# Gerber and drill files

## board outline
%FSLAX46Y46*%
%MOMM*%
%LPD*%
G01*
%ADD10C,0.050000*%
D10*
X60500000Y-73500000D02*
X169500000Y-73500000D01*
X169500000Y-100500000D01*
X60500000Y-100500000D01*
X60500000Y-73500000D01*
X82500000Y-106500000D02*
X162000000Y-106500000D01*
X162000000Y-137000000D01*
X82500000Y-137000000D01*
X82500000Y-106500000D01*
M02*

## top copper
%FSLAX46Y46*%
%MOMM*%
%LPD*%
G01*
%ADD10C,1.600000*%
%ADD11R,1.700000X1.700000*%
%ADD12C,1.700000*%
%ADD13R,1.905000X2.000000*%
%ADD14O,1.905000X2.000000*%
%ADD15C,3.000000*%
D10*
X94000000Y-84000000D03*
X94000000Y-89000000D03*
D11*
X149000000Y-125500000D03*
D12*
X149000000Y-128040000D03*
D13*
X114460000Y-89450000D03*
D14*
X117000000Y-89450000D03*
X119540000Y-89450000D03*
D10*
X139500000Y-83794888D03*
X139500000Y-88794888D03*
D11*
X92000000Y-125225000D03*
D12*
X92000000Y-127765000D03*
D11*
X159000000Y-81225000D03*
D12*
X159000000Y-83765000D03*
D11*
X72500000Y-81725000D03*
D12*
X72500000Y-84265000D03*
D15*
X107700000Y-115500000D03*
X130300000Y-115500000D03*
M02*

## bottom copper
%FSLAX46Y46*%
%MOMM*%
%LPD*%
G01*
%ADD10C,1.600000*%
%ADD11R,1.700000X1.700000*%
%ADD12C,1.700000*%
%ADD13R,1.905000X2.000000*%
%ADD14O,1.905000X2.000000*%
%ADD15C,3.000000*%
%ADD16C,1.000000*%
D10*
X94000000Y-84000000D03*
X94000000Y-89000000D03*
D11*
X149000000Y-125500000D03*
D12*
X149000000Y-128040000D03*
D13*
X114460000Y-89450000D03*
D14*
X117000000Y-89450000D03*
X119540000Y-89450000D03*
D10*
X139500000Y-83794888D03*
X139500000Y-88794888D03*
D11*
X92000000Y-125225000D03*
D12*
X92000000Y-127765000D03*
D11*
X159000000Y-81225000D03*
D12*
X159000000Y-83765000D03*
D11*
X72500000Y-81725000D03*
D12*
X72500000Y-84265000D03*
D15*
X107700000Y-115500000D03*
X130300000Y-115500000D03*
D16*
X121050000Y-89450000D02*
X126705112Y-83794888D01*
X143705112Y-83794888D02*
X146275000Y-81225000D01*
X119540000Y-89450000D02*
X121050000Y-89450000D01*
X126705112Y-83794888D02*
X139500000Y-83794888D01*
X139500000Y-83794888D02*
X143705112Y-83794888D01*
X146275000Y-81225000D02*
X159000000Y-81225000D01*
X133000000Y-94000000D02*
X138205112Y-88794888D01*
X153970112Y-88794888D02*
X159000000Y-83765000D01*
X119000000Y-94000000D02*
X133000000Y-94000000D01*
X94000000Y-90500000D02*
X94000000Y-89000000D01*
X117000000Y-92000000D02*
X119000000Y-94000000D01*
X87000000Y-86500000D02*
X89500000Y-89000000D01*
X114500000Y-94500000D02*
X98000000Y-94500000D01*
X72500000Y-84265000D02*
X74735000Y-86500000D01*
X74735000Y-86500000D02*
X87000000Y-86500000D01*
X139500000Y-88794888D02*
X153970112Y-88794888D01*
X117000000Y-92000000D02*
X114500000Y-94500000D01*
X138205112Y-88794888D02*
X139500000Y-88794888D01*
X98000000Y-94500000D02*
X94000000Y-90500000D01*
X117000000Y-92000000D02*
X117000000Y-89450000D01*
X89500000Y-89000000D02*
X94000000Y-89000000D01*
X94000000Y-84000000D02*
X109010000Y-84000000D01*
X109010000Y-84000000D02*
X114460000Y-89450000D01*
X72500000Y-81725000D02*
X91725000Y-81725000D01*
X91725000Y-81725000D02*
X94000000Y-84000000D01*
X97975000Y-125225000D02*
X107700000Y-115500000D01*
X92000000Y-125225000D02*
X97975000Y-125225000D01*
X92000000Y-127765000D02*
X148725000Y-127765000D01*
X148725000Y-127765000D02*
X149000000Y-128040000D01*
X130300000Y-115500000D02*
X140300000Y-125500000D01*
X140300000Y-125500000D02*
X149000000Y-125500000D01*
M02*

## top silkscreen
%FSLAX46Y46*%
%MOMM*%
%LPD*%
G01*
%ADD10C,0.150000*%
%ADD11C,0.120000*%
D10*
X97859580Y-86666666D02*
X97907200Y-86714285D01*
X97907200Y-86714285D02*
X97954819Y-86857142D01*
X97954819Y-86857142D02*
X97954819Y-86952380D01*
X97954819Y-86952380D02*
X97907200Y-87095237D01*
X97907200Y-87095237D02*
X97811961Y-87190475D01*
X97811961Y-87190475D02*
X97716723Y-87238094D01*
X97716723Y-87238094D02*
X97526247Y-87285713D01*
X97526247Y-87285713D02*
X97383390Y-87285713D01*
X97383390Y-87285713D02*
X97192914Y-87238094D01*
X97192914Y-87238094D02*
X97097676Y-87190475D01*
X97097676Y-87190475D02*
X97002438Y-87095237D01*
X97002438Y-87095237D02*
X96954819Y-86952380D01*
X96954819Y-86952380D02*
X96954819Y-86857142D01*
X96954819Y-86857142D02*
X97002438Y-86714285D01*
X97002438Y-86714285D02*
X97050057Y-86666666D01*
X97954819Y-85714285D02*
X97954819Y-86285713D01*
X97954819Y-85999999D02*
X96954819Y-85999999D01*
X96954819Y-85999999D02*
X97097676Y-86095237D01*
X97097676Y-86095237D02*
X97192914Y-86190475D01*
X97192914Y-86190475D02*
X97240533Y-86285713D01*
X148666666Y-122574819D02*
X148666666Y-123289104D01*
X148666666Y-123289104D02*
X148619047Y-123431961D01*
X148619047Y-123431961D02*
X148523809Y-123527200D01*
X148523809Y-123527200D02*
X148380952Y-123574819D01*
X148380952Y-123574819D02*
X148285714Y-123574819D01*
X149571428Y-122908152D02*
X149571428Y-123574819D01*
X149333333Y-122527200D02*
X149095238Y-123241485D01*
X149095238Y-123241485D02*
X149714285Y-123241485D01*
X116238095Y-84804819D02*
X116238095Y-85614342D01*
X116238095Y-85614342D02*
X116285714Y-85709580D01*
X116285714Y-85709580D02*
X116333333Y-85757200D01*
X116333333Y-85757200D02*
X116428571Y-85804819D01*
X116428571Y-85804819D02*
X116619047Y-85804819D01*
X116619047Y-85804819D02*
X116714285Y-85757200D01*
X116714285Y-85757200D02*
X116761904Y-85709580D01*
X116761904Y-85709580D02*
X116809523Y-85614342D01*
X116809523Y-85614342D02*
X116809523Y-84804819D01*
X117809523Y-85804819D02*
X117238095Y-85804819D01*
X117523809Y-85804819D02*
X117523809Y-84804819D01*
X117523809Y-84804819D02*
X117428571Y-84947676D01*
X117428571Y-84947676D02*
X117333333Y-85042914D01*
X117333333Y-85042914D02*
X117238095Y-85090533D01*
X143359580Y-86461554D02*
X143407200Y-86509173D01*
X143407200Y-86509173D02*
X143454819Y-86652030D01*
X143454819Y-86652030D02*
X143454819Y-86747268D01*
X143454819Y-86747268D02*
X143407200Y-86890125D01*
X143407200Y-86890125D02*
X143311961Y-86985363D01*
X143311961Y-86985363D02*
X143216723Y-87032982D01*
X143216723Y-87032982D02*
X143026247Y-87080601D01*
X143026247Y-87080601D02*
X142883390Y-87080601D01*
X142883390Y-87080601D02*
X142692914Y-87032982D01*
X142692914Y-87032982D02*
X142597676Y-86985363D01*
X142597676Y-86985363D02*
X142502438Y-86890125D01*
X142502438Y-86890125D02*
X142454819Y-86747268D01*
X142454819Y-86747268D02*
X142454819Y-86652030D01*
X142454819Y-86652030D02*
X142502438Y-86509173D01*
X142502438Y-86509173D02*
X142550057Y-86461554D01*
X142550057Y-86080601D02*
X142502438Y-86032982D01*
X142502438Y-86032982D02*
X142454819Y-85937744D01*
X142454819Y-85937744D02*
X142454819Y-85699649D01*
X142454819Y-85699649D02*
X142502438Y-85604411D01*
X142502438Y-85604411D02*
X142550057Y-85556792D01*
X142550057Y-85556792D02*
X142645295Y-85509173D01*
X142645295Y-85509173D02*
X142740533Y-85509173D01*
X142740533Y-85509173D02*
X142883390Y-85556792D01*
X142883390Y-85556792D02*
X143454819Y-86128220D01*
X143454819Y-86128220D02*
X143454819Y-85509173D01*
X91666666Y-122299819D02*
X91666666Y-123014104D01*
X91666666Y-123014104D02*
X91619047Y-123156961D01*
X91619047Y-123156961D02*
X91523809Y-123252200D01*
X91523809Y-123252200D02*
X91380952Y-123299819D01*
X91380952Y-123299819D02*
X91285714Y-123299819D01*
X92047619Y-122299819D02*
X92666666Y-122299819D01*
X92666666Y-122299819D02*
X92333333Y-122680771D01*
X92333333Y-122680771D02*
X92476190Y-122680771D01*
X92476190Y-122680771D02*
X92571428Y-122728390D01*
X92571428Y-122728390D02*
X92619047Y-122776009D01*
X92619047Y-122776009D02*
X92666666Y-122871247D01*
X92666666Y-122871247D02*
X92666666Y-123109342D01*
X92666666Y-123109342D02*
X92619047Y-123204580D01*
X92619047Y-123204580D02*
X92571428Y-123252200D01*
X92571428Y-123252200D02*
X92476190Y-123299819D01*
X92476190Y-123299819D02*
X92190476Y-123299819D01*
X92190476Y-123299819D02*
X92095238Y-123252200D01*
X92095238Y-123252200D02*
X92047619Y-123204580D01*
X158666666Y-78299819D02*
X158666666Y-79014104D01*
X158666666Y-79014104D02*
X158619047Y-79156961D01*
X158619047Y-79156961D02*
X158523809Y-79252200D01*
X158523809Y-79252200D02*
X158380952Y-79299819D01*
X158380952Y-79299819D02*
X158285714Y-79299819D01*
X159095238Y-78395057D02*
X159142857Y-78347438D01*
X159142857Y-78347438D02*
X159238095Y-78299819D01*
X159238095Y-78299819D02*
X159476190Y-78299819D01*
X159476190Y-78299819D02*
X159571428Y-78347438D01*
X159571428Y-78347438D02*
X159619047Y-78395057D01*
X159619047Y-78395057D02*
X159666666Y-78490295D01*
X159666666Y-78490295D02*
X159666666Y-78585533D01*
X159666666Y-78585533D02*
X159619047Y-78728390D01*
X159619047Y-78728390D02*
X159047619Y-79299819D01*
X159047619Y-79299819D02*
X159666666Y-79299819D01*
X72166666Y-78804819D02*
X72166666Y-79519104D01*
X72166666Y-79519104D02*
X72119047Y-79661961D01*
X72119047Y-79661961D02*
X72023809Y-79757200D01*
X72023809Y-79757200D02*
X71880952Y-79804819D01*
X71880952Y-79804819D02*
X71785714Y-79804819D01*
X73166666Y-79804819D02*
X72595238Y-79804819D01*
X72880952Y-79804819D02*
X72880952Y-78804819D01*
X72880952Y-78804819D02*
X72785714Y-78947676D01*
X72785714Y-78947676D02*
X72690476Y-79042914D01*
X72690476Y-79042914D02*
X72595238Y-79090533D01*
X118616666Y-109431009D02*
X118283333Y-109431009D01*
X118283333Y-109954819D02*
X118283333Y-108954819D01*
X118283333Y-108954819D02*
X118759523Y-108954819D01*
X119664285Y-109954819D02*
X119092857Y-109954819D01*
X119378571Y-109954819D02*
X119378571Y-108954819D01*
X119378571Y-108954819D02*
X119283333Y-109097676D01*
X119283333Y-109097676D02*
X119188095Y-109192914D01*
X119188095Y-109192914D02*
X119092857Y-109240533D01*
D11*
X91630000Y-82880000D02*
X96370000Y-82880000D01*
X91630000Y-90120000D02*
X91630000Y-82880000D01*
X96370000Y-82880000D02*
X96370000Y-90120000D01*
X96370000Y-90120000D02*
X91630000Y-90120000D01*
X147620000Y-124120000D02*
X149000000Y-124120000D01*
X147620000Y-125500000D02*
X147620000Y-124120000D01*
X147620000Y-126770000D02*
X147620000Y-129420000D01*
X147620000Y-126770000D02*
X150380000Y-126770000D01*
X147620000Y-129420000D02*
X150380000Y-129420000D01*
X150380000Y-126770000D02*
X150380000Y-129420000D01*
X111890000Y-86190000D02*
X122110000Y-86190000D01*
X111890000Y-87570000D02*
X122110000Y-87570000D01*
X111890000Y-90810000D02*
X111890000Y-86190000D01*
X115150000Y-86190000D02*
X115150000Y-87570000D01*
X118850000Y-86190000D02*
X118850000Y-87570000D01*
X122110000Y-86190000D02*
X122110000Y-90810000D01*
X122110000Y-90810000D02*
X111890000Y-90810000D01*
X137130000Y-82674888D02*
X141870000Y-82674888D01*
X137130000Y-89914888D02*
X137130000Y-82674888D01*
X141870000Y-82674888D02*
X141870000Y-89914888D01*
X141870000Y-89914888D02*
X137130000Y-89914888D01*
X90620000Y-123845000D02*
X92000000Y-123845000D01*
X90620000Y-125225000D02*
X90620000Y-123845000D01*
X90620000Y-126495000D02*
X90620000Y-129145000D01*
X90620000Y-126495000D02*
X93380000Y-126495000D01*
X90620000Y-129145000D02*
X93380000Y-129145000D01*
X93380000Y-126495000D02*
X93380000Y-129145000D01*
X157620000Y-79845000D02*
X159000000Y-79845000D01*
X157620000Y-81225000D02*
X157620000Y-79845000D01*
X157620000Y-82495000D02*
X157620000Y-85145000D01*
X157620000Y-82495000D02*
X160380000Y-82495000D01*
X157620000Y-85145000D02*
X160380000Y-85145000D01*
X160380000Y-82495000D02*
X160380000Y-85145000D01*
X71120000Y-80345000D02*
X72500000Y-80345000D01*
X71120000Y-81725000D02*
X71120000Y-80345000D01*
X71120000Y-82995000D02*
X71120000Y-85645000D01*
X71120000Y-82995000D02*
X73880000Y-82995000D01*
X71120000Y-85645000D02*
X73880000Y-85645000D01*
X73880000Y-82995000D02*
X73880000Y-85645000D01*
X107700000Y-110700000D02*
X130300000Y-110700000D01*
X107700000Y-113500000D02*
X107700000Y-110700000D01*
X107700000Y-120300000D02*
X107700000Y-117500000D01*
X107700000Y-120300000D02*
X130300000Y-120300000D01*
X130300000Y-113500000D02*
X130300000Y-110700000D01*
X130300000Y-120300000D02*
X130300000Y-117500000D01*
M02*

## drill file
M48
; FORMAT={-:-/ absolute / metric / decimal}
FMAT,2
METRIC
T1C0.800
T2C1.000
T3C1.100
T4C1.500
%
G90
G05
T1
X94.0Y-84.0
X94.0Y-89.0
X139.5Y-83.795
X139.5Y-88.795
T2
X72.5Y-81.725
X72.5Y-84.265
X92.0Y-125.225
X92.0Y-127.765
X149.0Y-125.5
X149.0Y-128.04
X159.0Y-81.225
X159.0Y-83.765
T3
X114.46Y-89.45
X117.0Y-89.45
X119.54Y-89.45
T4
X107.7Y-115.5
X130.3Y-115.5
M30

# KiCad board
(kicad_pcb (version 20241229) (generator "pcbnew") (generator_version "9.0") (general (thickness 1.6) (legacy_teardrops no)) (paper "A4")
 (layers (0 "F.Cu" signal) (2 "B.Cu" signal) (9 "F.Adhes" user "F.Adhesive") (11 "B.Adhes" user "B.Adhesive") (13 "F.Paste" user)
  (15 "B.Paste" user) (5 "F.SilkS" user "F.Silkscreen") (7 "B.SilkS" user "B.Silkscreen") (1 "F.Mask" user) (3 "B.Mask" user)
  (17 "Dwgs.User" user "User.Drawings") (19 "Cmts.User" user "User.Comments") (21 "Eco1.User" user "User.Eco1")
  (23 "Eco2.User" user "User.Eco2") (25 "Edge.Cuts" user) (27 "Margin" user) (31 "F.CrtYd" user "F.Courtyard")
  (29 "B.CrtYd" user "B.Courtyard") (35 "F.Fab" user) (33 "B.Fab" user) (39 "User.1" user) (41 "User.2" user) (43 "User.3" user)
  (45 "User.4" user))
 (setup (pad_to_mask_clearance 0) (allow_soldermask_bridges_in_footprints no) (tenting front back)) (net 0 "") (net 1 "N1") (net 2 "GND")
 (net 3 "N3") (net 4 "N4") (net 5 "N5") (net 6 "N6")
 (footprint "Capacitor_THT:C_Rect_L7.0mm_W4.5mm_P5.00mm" (layer "F.Cu") (at 94 84 -90)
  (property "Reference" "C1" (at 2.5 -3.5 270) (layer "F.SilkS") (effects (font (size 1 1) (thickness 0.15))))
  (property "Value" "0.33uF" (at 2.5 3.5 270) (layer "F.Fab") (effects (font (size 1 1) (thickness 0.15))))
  (fp_line (start -1.12 2.37) (end -1.12 -2.37) (stroke (width 0.12) (type solid)) (layer "F.SilkS"))
  (fp_line (start 6.12 2.37) (end -1.12 2.37) (stroke (width 0.12) (type solid)) (layer "F.SilkS"))
  (fp_line (start -1.12 -2.37) (end 6.12 -2.37) (stroke (width 0.12) (type solid)) (layer "F.SilkS"))
  (fp_line (start 6.12 -2.37) (end 6.12 2.37) (stroke (width 0.12) (type solid)) (layer "F.SilkS"))
  (pad "1" thru_hole circle (at 0 0 270) (size 1.6 1.6) (drill 0.8) (layers "*.Cu" "*.Mask") (remove_unused_layers no) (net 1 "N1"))
  (pad "2" thru_hole circle (at 5 0 270) (size 1.6 1.6) (drill 0.8) (layers "*.Cu" "*.Mask") (remove_unused_layers no) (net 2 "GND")))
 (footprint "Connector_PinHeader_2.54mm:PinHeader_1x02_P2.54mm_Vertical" (layer "F.Cu") (at 149 125.5)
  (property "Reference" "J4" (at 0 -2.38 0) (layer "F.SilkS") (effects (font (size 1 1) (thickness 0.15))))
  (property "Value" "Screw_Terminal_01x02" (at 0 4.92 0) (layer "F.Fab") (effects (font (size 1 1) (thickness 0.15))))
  (fp_line (start -1.38 -1.38) (end 0 -1.38) (stroke (width 0.12) (type solid)) (layer "F.SilkS"))
  (fp_line (start -1.38 0) (end -1.38 -1.38) (stroke (width 0.12) (type solid)) (layer "F.SilkS"))
  (fp_line (start -1.38 1.27) (end -1.38 3.92) (stroke (width 0.12) (type solid)) (layer "F.SilkS"))
  (fp_line (start -1.38 1.27) (end 1.38 1.27) (stroke (width 0.12) (type solid)) (layer "F.SilkS"))
  (fp_line (start -1.38 3.92) (end 1.38 3.92) (stroke (width 0.12) (type solid)) (layer "F.SilkS"))
  (fp_line (start 1.38 1.27) (end 1.38 3.92) (stroke (width 0.12) (type solid)) (layer "F.SilkS"))
  (pad "1" thru_hole rect (at 0 0) (size 1.7 1.7) (drill 1) (layers "*.Cu" "*.Mask") (remove_unused_layers no) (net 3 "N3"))
  (pad "2" thru_hole circle (at 0 2.54) (size 1.7 1.7) (drill 1) (layers "*.Cu" "*.Mask") (remove_unused_layers no) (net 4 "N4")))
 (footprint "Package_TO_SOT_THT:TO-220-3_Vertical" (layer "F.Cu") (at 114.46 89.45)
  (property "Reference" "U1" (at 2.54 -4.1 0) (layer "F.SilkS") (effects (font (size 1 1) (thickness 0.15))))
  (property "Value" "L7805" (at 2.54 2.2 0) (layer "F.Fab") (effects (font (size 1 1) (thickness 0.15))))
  (fp_line (start -2.57 -3.26) (end 7.65 -3.26) (stroke (width 0.12) (type solid)) (layer "F.SilkS"))
  (fp_line (start -2.57 -1.88) (end 7.65 -1.88) (stroke (width 0.12) (type solid)) (layer "F.SilkS"))
  (fp_line (start -2.57 1.36) (end -2.57 -3.26) (stroke (width 0.12) (type solid)) (layer "F.SilkS"))
  (fp_line (start 0.69 -3.26) (end 0.69 -1.88) (stroke (width 0.12) (type solid)) (layer "F.SilkS"))
  (fp_line (start 4.39 -3.26) (end 4.39 -1.88) (stroke (width 0.12) (type solid)) (layer "F.SilkS"))
  (fp_line (start 7.65 -3.26) (end 7.65 1.36) (stroke (width 0.12) (type solid)) (layer "F.SilkS"))
  (fp_line (start 7.65 1.36) (end -2.57 1.36) (stroke (width 0.12) (type solid)) (layer "F.SilkS"))
  (pad "1" thru_hole rect (at 0 0) (size 1.905 2) (drill 1.1) (layers "*.Cu" "*.Mask") (remove_unused_layers no) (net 1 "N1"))
  (pad "2" thru_hole oval (at 2.54 0) (size 1.905 2) (drill 1.1) (layers "*.Cu" "*.Mask") (remove_unused_layers no) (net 2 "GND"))
  (pad "3" thru_hole oval (at 5.08 0) (size 1.905 2) (drill 1.1) (layers "*.Cu" "*.Mask") (remove_unused_layers no) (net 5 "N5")))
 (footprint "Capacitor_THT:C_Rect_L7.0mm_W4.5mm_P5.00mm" (layer "F.Cu") (at 139.5 83.794888 -90)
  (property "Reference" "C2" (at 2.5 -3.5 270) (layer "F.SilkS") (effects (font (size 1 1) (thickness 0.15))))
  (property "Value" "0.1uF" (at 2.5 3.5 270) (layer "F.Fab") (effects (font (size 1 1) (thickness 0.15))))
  (fp_line (start -1.12 2.37) (end -1.12 -2.37) (stroke (width 0.12) (type solid)) (layer "F.SilkS"))
  (fp_line (start 6.12 2.37) (end -1.12 2.37) (stroke (width 0.12) (type solid)) (layer "F.SilkS"))
  (fp_line (start -1.12 -2.37) (end 6.12 -2.37) (stroke (width 0.12) (type solid)) (layer "F.SilkS"))
  (fp_line (start 6.12 -2.37) (end 6.12 2.37) (stroke (width 0.12) (type solid)) (layer "F.SilkS"))
  (pad "1" thru_hole circle (at 0 0 270) (size 1.6 1.6) (drill 0.8) (layers "*.Cu" "*.Mask") (remove_unused_layers no) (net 5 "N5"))
  (pad "2" thru_hole circle (at 5 0 270) (size 1.6 1.6) (drill 0.8) (layers "*.Cu" "*.Mask") (remove_unused_layers no) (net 2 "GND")))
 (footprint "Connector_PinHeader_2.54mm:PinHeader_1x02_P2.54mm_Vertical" (layer "F.Cu") (at 92 125.225)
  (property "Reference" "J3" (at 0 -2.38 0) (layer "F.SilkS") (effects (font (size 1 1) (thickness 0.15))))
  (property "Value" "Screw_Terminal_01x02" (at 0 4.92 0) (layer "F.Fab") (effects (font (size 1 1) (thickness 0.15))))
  (fp_line (start -1.38 -1.38) (end 0 -1.38) (stroke (width 0.12) (type solid)) (layer "F.SilkS"))
  (fp_line (start -1.38 0) (end -1.38 -1.38) (stroke (width 0.12) (type solid)) (layer "F.SilkS"))
  (fp_line (start -1.38 1.27) (end -1.38 3.92) (stroke (width 0.12) (type solid)) (layer "F.SilkS"))
  (fp_line (start -1.38 1.27) (end 1.38 1.27) (stroke (width 0.12) (type solid)) (layer "F.SilkS"))
  (fp_line (start -1.38 3.92) (end 1.38 3.92) (stroke (width 0.12) (type solid)) (layer "F.SilkS"))
  (fp_line (start 1.38 1.27) (end 1.38 3.92) (stroke (width 0.12) (type solid)) (layer "F.SilkS"))
  (pad "1" thru_hole rect (at 0 0) (size 1.7 1.7) (drill 1) (layers "*.Cu" "*.Mask") (remove_unused_layers no) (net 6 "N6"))
  (pad "2" thru_hole circle (at 0 2.54) (size 1.7 1.7) (drill 1) (layers "*.Cu" "*.Mask") (remove_unused_layers no) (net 4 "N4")))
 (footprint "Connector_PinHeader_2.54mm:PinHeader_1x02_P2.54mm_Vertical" (layer "F.Cu") (at 159 81.225)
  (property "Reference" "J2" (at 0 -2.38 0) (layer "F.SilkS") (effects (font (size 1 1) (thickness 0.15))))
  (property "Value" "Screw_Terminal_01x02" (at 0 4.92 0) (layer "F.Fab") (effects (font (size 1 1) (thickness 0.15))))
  (fp_line (start -1.38 -1.38) (end 0 -1.38) (stroke (width 0.12) (type solid)) (layer "F.SilkS"))
  (fp_line (start -1.38 0) (end -1.38 -1.38) (stroke (width 0.12) (type solid)) (layer "F.SilkS"))
  (fp_line (start -1.38 1.27) (end -1.38 3.92) (stroke (width 0.12) (type solid)) (layer "F.SilkS"))
  (fp_line (start -1.38 1.27) (end 1.38 1.27) (stroke (width 0.12) (type solid)) (layer "F.SilkS"))
  (fp_line (start -1.38 3.92) (end 1.38 3.92) (stroke (width 0.12) (type solid)) (layer "F.SilkS"))
  (fp_line (start 1.38 1.27) (end 1.38 3.92) (stroke (width 0.12) (type solid)) (layer "F.SilkS"))
  (pad "1" thru_hole rect (at 0 0) (size 1.7 1.7) (drill 1) (layers "*.Cu" "*.Mask") (remove_unused_layers no) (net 5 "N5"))
  (pad "2" thru_hole circle (at 0 2.54) (size 1.7 1.7) (drill 1) (layers "*.Cu" "*.Mask") (remove_unused_layers no) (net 2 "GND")))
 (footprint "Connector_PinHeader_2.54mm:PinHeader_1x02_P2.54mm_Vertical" (layer "F.Cu") (at 72.5 81.725)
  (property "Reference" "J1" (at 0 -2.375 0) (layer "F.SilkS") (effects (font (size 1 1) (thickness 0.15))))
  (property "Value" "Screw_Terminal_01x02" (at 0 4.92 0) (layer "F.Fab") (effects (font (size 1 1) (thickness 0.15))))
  (fp_line (start -1.38 -1.38) (end 0 -1.38) (stroke (width 0.12) (type solid)) (layer "F.SilkS"))
  (fp_line (start -1.38 0) (end -1.38 -1.38) (stroke (width 0.12) (type solid)) (layer "F.SilkS"))
  (fp_line (start -1.38 1.27) (end -1.38 3.92) (stroke (width 0.12) (type solid)) (layer "F.SilkS"))
  (fp_line (start -1.38 1.27) (end 1.38 1.27) (stroke (width 0.12) (type solid)) (layer "F.SilkS"))
  (fp_line (start -1.38 3.92) (end 1.38 3.92) (stroke (width 0.12) (type solid)) (layer "F.SilkS"))
  (fp_line (start 1.38 1.27) (end 1.38 3.92) (stroke (width 0.12) (type solid)) (layer "F.SilkS"))
  (pad "1" thru_hole rect (at 0 0) (size 1.7 1.7) (drill 1) (layers "*.Cu" "*.Mask") (remove_unused_layers no) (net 1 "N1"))
  (pad "2" thru_hole circle (at 0 2.54) (size 1.7 1.7) (drill 1) (layers "*.Cu" "*.Mask") (remove_unused_layers no) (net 2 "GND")))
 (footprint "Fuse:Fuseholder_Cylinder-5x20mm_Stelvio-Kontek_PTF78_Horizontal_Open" (layer "F.Cu") (at 107.7 115.5)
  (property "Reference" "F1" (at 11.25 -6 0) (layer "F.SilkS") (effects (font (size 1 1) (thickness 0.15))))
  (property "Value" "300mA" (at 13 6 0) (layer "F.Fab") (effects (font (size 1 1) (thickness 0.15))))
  (fp_line (start 0 -4.8) (end 22.6 -4.8) (stroke (width 0.12) (type solid)) (layer "F.SilkS"))
  (fp_line (start 0 -2) (end 0 -4.8) (stroke (width 0.12) (type solid)) (layer "F.SilkS"))
  (fp_line (start 0 4.8) (end 0 2) (stroke (width 0.12) (type solid)) (layer "F.SilkS"))
  (fp_line (start 0 4.8) (end 22.6 4.8) (stroke (width 0.12) (type solid)) (layer "F.SilkS"))
  (fp_line (start 22.6 -2) (end 22.6 -4.8) (stroke (width 0.12) (type solid)) (layer "F.SilkS"))
  (fp_line (start 22.6 4.8) (end 22.6 2) (stroke (width 0.12) (type solid)) (layer "F.SilkS"))
  (pad "1" thru_hole circle (at 0 0) (size 3 3) (drill 1.5) (layers "*.Cu" "*.Mask") (remove_unused_layers no) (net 6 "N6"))
  (pad "2" thru_hole circle (at 22.6 0) (size 3 3) (drill 1.5) (layers "*.Cu" "*.Mask") (remove_unused_layers no) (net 3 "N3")))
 (gr_rect (start 60.5 73.5) (end 169.5 100.5) (stroke (width 0.05) (type default)) (fill no) (layer "Edge.Cuts"))
 (gr_rect (start 82.5 106.5) (end 162 137) (stroke (width 0.05) (type default)) (fill no) (layer "Edge.Cuts"))
 (segment (start 121.05 89.45) (end 126.705112 83.794888) (width 1) (layer "B.Cu") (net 5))
 (segment (start 143.705112 83.794888) (end 146.275 81.225) (width 1) (layer "B.Cu") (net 5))
 (segment (start 119.54 89.45) (end 121.05 89.45) (width 1) (layer "B.Cu") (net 5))
 (segment (start 126.705112 83.794888) (end 139.5 83.794888) (width 1) (layer "B.Cu") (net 5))
 (segment (start 139.5 83.794888) (end 143.705112 83.794888) (width 1) (layer "B.Cu") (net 5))
 (segment (start 146.275 81.225) (end 159 81.225) (width 1) (layer "B.Cu") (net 5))
 (segment (start 133 94) (end 138.205112 88.794888) (width 1) (layer "B.Cu") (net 2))
 (segment (start 153.970112 88.794888) (end 159 83.765) (width 1) (layer "B.Cu") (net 2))
 (segment (start 119 94) (end 133 94) (width 1) (layer "B.Cu") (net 2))
 (segment (start 94 90.5) (end 94 89) (width 1) (layer "B.Cu") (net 2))
 (segment (start 117 92) (end 119 94) (width 1) (layer "B.Cu") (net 2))
 (segment (start 87 86.5) (end 89.5 89) (width 1) (layer "B.Cu") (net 2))
 (segment (start 114.5 94.5) (end 98 94.5) (width 1) (layer "B.Cu") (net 2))
 (segment (start 72.5 84.265) (end 74.735 86.5) (width 1) (layer "B.Cu") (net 2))
 (segment (start 74.735 86.5) (end 87 86.5) (width 1) (layer "B.Cu") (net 2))
 (segment (start 139.5 88.794888) (end 153.970112 88.794888) (width 1) (layer "B.Cu") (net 2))
 (segment (start 117 92) (end 114.5 94.5) (width 1) (layer "B.Cu") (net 2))
 (segment (start 138.205112 88.794888) (end 139.5 88.794888) (width 1) (layer "B.Cu") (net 2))
 (segment (start 98 94.5) (end 94 90.5) (width 1) (layer "B.Cu") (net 2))
 (segment (start 117 92) (end 117 89.45) (width 1) (layer "B.Cu") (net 2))
 (segment (start 89.5 89) (end 94 89) (width 1) (layer "B.Cu") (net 2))
 (segment (start 94 84) (end 109.01 84) (width 1) (layer "B.Cu") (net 1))
 (segment (start 109.01 84) (end 114.46 89.45) (width 1) (layer "B.Cu") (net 1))
 (segment (start 72.5 81.725) (end 91.725 81.725) (width 1) (layer "B.Cu") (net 1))
 (segment (start 91.725 81.725) (end 94 84) (width 1) (layer "B.Cu") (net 1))
 (segment (start 97.975 125.225) (end 107.7 115.5) (width 1) (layer "B.Cu") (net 6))
 (segment (start 92 125.225) (end 97.975 125.225) (width 1) (layer "B.Cu") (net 6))
 (segment (start 92 127.765) (end 148.725 127.765) (width 1) (layer "B.Cu") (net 4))
 (segment (start 148.725 127.765) (end 149 128.04) (width 1) (layer "B.Cu") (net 4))
 (segment (start 130.3 115.5) (end 140.3 125.5) (width 1) (layer "B.Cu") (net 3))
 (segment (start 140.3 125.5) (end 149 125.5) (width 1) (layer "B.Cu") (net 3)))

